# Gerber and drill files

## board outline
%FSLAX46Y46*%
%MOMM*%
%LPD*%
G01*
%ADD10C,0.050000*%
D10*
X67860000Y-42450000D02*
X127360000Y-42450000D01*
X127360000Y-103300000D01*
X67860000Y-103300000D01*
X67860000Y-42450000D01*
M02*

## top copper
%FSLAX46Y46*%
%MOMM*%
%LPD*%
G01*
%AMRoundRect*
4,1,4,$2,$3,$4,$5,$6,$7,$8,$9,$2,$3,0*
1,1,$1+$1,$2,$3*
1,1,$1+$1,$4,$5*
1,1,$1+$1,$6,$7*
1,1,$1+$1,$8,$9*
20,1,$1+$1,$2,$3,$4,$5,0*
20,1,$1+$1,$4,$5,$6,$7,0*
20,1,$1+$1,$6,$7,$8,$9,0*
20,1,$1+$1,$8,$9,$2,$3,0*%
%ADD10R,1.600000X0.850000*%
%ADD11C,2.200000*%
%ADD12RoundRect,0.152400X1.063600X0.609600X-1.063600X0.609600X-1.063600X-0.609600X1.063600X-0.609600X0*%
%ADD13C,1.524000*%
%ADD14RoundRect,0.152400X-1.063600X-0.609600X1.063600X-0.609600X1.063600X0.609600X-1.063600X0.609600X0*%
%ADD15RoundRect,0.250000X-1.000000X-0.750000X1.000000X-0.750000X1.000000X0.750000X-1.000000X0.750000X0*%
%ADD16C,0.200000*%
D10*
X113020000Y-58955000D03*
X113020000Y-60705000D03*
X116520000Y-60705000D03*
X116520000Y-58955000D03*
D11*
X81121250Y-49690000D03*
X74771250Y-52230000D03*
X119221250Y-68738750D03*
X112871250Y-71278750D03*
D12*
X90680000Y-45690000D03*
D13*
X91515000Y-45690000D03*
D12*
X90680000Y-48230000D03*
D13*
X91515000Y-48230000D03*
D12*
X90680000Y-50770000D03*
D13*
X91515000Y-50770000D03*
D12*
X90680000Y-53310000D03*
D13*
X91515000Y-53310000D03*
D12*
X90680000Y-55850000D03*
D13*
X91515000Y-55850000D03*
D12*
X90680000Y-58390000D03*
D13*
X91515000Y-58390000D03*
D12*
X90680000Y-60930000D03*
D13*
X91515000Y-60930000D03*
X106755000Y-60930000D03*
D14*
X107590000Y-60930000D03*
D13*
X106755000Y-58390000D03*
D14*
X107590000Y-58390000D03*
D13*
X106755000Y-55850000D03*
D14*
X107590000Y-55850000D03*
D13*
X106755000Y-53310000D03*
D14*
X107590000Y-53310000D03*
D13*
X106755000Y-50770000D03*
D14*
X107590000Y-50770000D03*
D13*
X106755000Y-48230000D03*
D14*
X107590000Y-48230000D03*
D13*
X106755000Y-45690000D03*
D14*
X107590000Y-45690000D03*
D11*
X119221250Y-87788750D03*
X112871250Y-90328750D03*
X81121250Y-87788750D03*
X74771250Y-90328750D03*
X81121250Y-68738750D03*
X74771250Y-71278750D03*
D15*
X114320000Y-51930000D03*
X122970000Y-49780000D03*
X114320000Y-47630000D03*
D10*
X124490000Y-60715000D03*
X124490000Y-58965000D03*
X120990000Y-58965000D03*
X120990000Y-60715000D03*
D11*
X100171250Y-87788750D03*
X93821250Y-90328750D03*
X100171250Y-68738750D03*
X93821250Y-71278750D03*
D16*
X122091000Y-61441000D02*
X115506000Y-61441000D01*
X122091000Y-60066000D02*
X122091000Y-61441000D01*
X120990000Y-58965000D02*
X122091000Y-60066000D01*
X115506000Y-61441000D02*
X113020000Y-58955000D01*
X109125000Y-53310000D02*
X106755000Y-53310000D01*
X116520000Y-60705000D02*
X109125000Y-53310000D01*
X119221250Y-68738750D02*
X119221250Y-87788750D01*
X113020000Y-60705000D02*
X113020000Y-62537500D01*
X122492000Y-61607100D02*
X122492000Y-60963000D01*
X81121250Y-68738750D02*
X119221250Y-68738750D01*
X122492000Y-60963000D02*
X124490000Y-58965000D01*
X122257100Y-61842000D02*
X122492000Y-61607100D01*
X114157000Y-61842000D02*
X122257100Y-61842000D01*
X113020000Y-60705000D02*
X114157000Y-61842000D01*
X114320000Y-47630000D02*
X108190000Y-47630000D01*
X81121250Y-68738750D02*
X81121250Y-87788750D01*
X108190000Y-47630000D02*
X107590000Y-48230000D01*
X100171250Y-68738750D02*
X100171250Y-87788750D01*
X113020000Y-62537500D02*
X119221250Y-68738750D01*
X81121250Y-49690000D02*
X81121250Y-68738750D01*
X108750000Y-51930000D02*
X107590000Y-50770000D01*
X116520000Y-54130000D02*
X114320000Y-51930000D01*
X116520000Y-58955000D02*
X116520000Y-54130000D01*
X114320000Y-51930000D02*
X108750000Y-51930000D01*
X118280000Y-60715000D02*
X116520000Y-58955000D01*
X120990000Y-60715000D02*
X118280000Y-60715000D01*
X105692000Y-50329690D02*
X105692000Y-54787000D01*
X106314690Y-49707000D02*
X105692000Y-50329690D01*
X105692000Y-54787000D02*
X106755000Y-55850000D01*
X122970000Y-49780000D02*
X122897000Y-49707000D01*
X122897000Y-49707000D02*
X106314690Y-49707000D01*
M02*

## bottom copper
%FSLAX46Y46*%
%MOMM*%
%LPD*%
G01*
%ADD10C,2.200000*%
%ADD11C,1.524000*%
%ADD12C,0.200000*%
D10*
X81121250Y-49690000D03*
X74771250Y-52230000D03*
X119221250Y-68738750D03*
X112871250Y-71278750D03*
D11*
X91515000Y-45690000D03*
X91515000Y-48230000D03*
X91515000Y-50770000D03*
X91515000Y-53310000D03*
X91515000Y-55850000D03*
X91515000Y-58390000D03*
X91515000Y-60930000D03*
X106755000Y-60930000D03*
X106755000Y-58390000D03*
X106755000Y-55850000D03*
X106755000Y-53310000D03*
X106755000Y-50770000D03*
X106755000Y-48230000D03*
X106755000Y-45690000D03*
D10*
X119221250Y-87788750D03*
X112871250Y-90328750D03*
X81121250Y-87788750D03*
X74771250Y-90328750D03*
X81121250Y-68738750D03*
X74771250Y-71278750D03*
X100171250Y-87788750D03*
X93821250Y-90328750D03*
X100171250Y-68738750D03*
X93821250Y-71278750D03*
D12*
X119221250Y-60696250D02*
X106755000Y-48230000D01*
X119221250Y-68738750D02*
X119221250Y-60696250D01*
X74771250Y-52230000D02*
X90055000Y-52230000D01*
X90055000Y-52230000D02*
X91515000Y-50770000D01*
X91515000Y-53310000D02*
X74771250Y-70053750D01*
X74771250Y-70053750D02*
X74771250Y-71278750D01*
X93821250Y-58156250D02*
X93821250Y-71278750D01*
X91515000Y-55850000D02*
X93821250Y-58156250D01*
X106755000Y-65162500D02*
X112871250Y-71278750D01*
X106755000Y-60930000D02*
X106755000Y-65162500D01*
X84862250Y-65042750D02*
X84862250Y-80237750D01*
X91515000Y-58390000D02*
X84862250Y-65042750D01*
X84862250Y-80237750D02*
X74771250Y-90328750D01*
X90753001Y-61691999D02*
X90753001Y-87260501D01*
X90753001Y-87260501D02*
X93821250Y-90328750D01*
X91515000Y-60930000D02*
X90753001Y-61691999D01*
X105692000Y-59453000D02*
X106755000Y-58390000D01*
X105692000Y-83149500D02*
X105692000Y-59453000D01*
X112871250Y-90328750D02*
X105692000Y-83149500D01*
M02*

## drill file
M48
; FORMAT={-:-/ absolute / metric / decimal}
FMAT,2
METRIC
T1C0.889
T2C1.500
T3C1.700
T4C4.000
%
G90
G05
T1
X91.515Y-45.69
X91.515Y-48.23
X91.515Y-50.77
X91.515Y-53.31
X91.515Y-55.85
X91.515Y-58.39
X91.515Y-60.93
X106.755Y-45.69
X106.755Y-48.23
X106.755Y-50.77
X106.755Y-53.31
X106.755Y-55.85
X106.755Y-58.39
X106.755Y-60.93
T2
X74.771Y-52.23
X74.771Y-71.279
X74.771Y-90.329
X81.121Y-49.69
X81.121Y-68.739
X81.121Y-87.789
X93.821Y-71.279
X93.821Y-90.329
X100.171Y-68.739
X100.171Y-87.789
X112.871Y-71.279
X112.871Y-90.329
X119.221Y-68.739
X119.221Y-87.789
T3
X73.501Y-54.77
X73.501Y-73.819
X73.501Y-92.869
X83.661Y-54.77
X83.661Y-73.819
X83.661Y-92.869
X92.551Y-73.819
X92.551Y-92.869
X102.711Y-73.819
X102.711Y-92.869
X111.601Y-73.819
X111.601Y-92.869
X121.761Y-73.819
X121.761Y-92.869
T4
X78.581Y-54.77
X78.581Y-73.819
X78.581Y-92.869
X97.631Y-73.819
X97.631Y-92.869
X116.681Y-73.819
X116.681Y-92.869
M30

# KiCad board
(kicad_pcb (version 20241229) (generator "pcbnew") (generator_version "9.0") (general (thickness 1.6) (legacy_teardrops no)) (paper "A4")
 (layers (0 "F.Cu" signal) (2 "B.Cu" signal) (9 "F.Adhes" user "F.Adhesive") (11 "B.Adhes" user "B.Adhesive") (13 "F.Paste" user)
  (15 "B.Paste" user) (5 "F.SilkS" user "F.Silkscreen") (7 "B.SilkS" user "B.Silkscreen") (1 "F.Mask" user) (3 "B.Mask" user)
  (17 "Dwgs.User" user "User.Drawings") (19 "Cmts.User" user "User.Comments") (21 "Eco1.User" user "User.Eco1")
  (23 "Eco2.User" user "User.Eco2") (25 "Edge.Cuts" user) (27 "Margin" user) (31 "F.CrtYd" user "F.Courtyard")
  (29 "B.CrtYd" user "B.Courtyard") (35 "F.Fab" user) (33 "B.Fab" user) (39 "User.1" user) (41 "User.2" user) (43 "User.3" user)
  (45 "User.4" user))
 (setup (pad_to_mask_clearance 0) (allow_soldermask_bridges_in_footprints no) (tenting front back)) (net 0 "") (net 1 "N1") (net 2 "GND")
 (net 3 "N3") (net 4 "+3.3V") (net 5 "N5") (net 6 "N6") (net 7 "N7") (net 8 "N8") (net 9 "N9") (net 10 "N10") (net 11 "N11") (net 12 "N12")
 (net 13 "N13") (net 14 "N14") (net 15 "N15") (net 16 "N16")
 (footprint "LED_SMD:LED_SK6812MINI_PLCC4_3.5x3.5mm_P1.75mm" (layer "F.Cu") (at 114.77 59.83)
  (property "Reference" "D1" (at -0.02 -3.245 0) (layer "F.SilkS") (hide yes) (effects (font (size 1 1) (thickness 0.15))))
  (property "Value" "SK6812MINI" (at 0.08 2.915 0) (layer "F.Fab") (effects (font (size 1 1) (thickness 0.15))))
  (pad "1" smd rect (at -1.75 -0.875) (size 1.6 0.85) (layers "F.Cu" "F.Mask" "F.Paste") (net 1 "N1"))
  (pad "2" smd rect (at -1.75 0.875) (size 1.6 0.85) (layers "F.Cu" "F.Mask" "F.Paste") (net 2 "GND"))
  (pad "3" smd rect (at 1.75 0.875) (size 1.6 0.85) (layers "F.Cu" "F.Mask" "F.Paste") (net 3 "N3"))
  (pad "4" smd rect (at 1.75 -0.875) (size 1.6 0.85) (layers "F.Cu" "F.Mask" "F.Paste") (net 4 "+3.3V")))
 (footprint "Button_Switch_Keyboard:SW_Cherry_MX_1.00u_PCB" (layer "F.Cu") (at 81.12125 49.69)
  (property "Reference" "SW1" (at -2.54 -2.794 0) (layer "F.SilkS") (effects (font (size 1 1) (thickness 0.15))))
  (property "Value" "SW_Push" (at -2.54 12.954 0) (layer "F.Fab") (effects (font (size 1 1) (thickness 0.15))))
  (pad "" np_thru_hole circle (at -7.62 5.08) (size 1.7 1.7) (drill 1.7) (layers "*.Cu" "*.Mask"))
  (pad "" np_thru_hole circle (at -2.54 5.08) (size 4 4) (drill 4) (layers "*.Cu" "*.Mask"))
  (pad "" np_thru_hole circle (at 2.54 5.08) (size 1.7 1.7) (drill 1.7) (layers "*.Cu" "*.Mask"))
  (pad "1" thru_hole circle (at 0 0) (size 2.2 2.2) (drill 1.5) (layers "*.Cu" "*.Mask") (remove_unused_layers no) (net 2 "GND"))
  (pad "2" thru_hole circle (at -6.35 2.54) (size 2.2 2.2) (drill 1.5) (layers "*.Cu" "*.Mask") (remove_unused_layers no) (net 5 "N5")))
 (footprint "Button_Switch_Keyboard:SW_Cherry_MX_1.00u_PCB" (layer "F.Cu") (at 119.22125 68.73875)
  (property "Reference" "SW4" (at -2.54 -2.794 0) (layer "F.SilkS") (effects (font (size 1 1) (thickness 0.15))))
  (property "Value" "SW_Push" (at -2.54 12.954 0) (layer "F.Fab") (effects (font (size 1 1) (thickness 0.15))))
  (pad "" np_thru_hole circle (at -7.62 5.08) (size 1.7 1.7) (drill 1.7) (layers "*.Cu" "*.Mask"))
  (pad "" np_thru_hole circle (at -2.54 5.08) (size 4 4) (drill 4) (layers "*.Cu" "*.Mask"))
  (pad "" np_thru_hole circle (at 2.54 5.08) (size 1.7 1.7) (drill 1.7) (layers "*.Cu" "*.Mask"))
  (pad "1" thru_hole circle (at 0 0) (size 2.2 2.2) (drill 1.5) (layers "*.Cu" "*.Mask") (remove_unused_layers no) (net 2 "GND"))
  (pad "2" thru_hole circle (at -6.35 2.54) (size 2.2 2.2) (drill 1.5) (layers "*.Cu" "*.Mask") (remove_unused_layers no) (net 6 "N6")))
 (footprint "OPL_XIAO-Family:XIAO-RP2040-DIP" (layer "F.Cu") (at 99.135 53.31)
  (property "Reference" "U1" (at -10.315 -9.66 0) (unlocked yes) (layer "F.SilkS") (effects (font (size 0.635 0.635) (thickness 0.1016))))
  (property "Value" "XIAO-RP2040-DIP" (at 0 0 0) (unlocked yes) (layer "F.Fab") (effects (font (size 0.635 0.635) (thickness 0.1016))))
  (pad "1" smd roundrect (at -8.455 -7.62 180) (size 2.432 1.524) (layers "F.Cu" "F.Mask") (roundrect_rratio 0.1) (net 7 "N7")
   (thermal_bridge_angle 45))
  (pad "1" thru_hole circle (at -7.62 -7.62 180) (size 1.524 1.524) (drill 0.889) (layers "*.Cu" "*.Mask") (remove_unused_layers no)
   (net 7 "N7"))
  (pad "2" smd roundrect (at -8.455 -5.08 180) (size 2.432 1.524) (layers "F.Cu" "F.Mask") (roundrect_rratio 0.1) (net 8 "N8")
   (thermal_bridge_angle 45))
  (pad "2" thru_hole circle (at -7.62 -5.08 180) (size 1.524 1.524) (drill 0.889) (layers "*.Cu" "*.Mask") (remove_unused_layers no)
   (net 8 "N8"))
  (pad "3" smd roundrect (at -8.455 -2.54 180) (size 2.432 1.524) (layers "F.Cu" "F.Mask") (roundrect_rratio 0.1) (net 5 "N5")
   (thermal_bridge_angle 45))
  (pad "3" thru_hole circle (at -7.62 -2.54 180) (size 1.524 1.524) (drill 0.889) (layers "*.Cu" "*.Mask") (remove_unused_layers no)
   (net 5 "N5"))
  (pad "4" smd roundrect (at -8.455 0 180) (size 2.432 1.524) (layers "F.Cu" "F.Mask") (roundrect_rratio 0.1) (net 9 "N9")
   (thermal_bridge_angle 45))
  (pad "4" thru_hole circle (at -7.62 0 180) (size 1.524 1.524) (drill 0.889) (layers "*.Cu" "*.Mask") (remove_unused_layers no)
   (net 9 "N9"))
  (pad "5" smd roundrect (at -8.455 2.54 180) (size 2.432 1.524) (layers "F.Cu" "F.Mask") (roundrect_rratio 0.1) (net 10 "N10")
   (thermal_bridge_angle 45))
  (pad "5" thru_hole circle (at -7.62 2.54 180) (size 1.524 1.524) (drill 0.889) (layers "*.Cu" "*.Mask") (remove_unused_layers no)
   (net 10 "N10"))
  (pad "6" smd roundrect (at -8.455 5.08 180) (size 2.432 1.524) (layers "F.Cu" "F.Mask") (roundrect_rratio 0.1) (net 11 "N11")
   (thermal_bridge_angle 45))
  (pad "6" thru_hole circle (at -7.62 5.08 180) (size 1.524 1.524) (drill 0.889) (layers "*.Cu" "*.Mask") (remove_unused_layers no)
   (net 11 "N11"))
  (pad "7" smd roundrect (at -8.455 7.62 180) (size 2.432 1.524) (layers "F.Cu" "F.Mask") (roundrect_rratio 0.1) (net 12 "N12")
   (thermal_bridge_angle 45))
  (pad "7" thru_hole circle (at -7.62 7.62 180) (size 1.524 1.524) (drill 0.889) (layers "*.Cu" "*.Mask") (remove_unused_layers no)
   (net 12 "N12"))
  (pad "8" thru_hole circle (at 7.62 7.62) (size 1.524 1.524) (drill 0.889) (layers "*.Cu" "*.Mask") (remove_unused_layers no) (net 6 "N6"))
  (pad "8" smd roundrect (at 8.455 7.62) (size 2.432 1.524) (layers "F.Cu" "F.Mask") (roundrect_rratio 0.1) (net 6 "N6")
   (thermal_bridge_angle 45))
  (pad "9" thru_hole circle (at 7.62 5.08) (size 1.524 1.524) (drill 0.889) (layers "*.Cu" "*.Mask") (remove_unused_layers no)
   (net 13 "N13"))
  (pad "9" smd roundrect (at 8.455 5.08) (size 2.432 1.524) (layers "F.Cu" "F.Mask") (roundrect_rratio 0.1) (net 13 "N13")
   (thermal_bridge_angle 45))
  (pad "10" thru_hole circle (at 7.62 2.54) (size 1.524 1.524) (drill 0.889) (layers "*.Cu" "*.Mask") (remove_unused_layers no)
   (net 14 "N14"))
  (pad "10" smd roundrect (at 8.455 2.54) (size 2.432 1.524) (layers "F.Cu" "F.Mask") (roundrect_rratio 0.1) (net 14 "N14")
   (thermal_bridge_angle 45))
  (pad "11" thru_hole circle (at 7.62 0) (size 1.524 1.524) (drill 0.889) (layers "*.Cu" "*.Mask") (remove_unused_layers no) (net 3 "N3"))
  (pad "11" smd roundrect (at 8.455 0) (size 2.432 1.524) (layers "F.Cu" "F.Mask") (roundrect_rratio 0.1) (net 3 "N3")
   (thermal_bridge_angle 45))
  (pad "12" thru_hole circle (at 7.62 -2.54) (size 1.524 1.524) (drill 0.889) (layers "*.Cu" "*.Mask") (remove_unused_layers no)
   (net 4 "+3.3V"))
  (pad "12" smd roundrect (at 8.455 -2.54) (size 2.432 1.524) (layers "F.Cu" "F.Mask") (roundrect_rratio 0.1) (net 4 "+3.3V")
   (thermal_bridge_angle 45))
  (pad "13" thru_hole circle (at 7.62 -5.08) (size 1.524 1.524) (drill 0.889) (layers "*.Cu" "*.Mask") (remove_unused_layers no)
   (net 2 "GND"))
  (pad "13" smd roundrect (at 8.455 -5.08) (size 2.432 1.524) (layers "F.Cu" "F.Mask") (roundrect_rratio 0.1) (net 2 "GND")
   (thermal_bridge_angle 45))
  (pad "14" thru_hole circle (at 7.62 -7.62) (size 1.524 1.524) (drill 0.889) (layers "*.Cu" "*.Mask") (remove_unused_layers no)
   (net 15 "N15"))
  (pad "14" smd roundrect (at 8.455 -7.62) (size 2.432 1.524) (layers "F.Cu" "F.Mask") (roundrect_rratio 0.1) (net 15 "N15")
   (thermal_bridge_angle 45)))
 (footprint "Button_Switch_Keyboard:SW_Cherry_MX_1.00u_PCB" (layer "F.Cu") (at 119.22125 87.78875)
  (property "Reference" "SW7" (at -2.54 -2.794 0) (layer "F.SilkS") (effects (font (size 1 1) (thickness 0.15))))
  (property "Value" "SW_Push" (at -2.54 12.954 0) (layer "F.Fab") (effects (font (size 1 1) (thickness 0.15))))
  (pad "" np_thru_hole circle (at -7.62 5.08) (size 1.7 1.7) (drill 1.7) (layers "*.Cu" "*.Mask"))
  (pad "" np_thru_hole circle (at -2.54 5.08) (size 4 4) (drill 4) (layers "*.Cu" "*.Mask"))
  (pad "" np_thru_hole circle (at 2.54 5.08) (size 1.7 1.7) (drill 1.7) (layers "*.Cu" "*.Mask"))
  (pad "1" thru_hole circle (at 0 0) (size 2.2 2.2) (drill 1.5) (layers "*.Cu" "*.Mask") (remove_unused_layers no) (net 2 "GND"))
  (pad "2" thru_hole circle (at -6.35 2.54) (size 2.2 2.2) (drill 1.5) (layers "*.Cu" "*.Mask") (remove_unused_layers no) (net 13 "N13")))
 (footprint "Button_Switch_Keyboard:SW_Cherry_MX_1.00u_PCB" (layer "F.Cu") (at 81.12125 87.78875)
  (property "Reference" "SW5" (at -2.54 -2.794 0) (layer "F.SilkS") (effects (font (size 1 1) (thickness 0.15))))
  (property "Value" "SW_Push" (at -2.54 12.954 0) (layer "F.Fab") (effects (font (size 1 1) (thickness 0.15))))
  (pad "" np_thru_hole circle (at -7.62 5.08) (size 1.7 1.7) (drill 1.7) (layers "*.Cu" "*.Mask"))
  (pad "" np_thru_hole circle (at -2.54 5.08) (size 4 4) (drill 4) (layers "*.Cu" "*.Mask"))
  (pad "" np_thru_hole circle (at 2.54 5.08) (size 1.7 1.7) (drill 1.7) (layers "*.Cu" "*.Mask"))
  (pad "1" thru_hole circle (at 0 0) (size 2.2 2.2) (drill 1.5) (layers "*.Cu" "*.Mask") (remove_unused_layers no) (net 2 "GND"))
  (pad "2" thru_hole circle (at -6.35 2.54) (size 2.2 2.2) (drill 1.5) (layers "*.Cu" "*.Mask") (remove_unused_layers no) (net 11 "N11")))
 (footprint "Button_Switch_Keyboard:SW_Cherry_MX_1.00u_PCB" (layer "F.Cu") (at 81.12125 68.73875)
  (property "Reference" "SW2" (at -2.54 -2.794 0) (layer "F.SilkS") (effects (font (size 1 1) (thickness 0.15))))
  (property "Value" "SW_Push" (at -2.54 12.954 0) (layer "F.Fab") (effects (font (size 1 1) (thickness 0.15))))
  (pad "" np_thru_hole circle (at -7.62 5.08) (size 1.7 1.7) (drill 1.7) (layers "*.Cu" "*.Mask"))
  (pad "" np_thru_hole circle (at -2.54 5.08) (size 4 4) (drill 4) (layers "*.Cu" "*.Mask"))
  (pad "" np_thru_hole circle (at 2.54 5.08) (size 1.7 1.7) (drill 1.7) (layers "*.Cu" "*.Mask"))
  (pad "1" thru_hole circle (at 0 0) (size 2.2 2.2) (drill 1.5) (layers "*.Cu" "*.Mask") (remove_unused_layers no) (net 2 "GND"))
  (pad "2" thru_hole circle (at -6.35 2.54) (size 2.2 2.2) (drill 1.5) (layers "*.Cu" "*.Mask") (remove_unused_layers no) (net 9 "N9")))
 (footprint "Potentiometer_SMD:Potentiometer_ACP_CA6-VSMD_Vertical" (layer "F.Cu") (at 118.645 49.78)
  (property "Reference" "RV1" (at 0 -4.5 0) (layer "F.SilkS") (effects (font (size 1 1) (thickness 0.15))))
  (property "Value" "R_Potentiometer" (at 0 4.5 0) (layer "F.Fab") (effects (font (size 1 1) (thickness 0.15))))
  (pad "1" smd roundrect (at -4.325 2.15) (size 2.5 2) (layers "F.Cu" "F.Mask" "F.Paste") (roundrect_rratio 0.125) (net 4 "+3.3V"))
  (pad "2" smd roundrect (at 4.325 0) (size 2.5 2) (layers "F.Cu" "F.Mask" "F.Paste") (roundrect_rratio 0.125) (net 14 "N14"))
  (pad "3" smd roundrect (at -4.325 -2.15) (size 2.5 2) (layers "F.Cu" "F.Mask" "F.Paste") (roundrect_rratio 0.125) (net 2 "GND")))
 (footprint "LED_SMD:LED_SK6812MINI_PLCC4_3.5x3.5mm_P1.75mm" (layer "F.Cu") (at 122.74 59.84 180)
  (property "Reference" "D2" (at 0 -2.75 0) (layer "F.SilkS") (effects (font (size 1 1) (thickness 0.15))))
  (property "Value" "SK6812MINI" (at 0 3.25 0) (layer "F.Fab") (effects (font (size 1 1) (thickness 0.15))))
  (pad "1" smd rect (at -1.75 -0.875 180) (size 1.6 0.85) (layers "F.Cu" "F.Mask" "F.Paste") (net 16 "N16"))
  (pad "2" smd rect (at -1.75 0.875 180) (size 1.6 0.85) (layers "F.Cu" "F.Mask" "F.Paste") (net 2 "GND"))
  (pad "3" smd rect (at 1.75 0.875 180) (size 1.6 0.85) (layers "F.Cu" "F.Mask" "F.Paste") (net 1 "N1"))
  (pad "4" smd rect (at 1.75 -0.875 180) (size 1.6 0.85) (layers "F.Cu" "F.Mask" "F.Paste") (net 4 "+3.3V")))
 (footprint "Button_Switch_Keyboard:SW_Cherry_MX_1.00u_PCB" (layer "F.Cu") (at 100.17125 87.78875)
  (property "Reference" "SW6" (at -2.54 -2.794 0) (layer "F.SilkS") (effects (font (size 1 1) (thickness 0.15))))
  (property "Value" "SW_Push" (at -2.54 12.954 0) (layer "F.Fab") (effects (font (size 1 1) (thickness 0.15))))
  (pad "" np_thru_hole circle (at -7.62 5.08) (size 1.7 1.7) (drill 1.7) (layers "*.Cu" "*.Mask"))
  (pad "" np_thru_hole circle (at -2.54 5.08) (size 4 4) (drill 4) (layers "*.Cu" "*.Mask"))
  (pad "" np_thru_hole circle (at 2.54 5.08) (size 1.7 1.7) (drill 1.7) (layers "*.Cu" "*.Mask"))
  (pad "1" thru_hole circle (at 0 0) (size 2.2 2.2) (drill 1.5) (layers "*.Cu" "*.Mask") (remove_unused_layers no) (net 2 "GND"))
  (pad "2" thru_hole circle (at -6.35 2.54) (size 2.2 2.2) (drill 1.5) (layers "*.Cu" "*.Mask") (remove_unused_layers no) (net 12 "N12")))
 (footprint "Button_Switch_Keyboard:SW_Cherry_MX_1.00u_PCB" (layer "F.Cu") (at 100.17125 68.73875)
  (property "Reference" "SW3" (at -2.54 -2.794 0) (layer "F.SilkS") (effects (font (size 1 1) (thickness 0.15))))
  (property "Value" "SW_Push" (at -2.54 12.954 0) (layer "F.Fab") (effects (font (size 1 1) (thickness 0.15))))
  (pad "" np_thru_hole circle (at -7.62 5.08) (size 1.7 1.7) (drill 1.7) (layers "*.Cu" "*.Mask"))
  (pad "" np_thru_hole circle (at -2.54 5.08) (size 4 4) (drill 4) (layers "*.Cu" "*.Mask"))
  (pad "" np_thru_hole circle (at 2.54 5.08) (size 1.7 1.7) (drill 1.7) (layers "*.Cu" "*.Mask"))
  (pad "1" thru_hole circle (at 0 0) (size 2.2 2.2) (drill 1.5) (layers "*.Cu" "*.Mask") (remove_unused_layers no) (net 2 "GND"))
  (pad "2" thru_hole circle (at -6.35 2.54) (size 2.2 2.2) (drill 1.5) (layers "*.Cu" "*.Mask") (remove_unused_layers no) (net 10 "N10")))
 (gr_rect (start 67.86 42.45) (end 127.36 103.3) (stroke (width 0.05) (type default)) (fill no) (layer "Edge.Cuts"))
 (segment (start 122.091 61.441) (end 115.506 61.441) (width 0.2) (layer "F.Cu") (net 1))
 (segment (start 122.091 60.066) (end 122.091 61.441) (width 0.2) (layer "F.Cu") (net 1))
 (segment (start 120.99 58.965) (end 122.091 60.066) (width 0.2) (layer "F.Cu") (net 1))
 (segment (start 115.506 61.441) (end 113.02 58.955) (width 0.2) (layer "F.Cu") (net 1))
 (segment (start 109.125 53.31) (end 106.755 53.31) (width 0.2) (layer "F.Cu") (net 3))
 (segment (start 116.52 60.705) (end 109.125 53.31) (width 0.2) (layer "F.Cu") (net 3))
 (segment (start 119.22125 68.73875) (end 119.22125 87.78875) (width 0.2) (layer "F.Cu") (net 2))
 (segment (start 113.02 60.705) (end 113.02 62.5375) (width 0.2) (layer "F.Cu") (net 2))
 (segment (start 122.492 61.6071) (end 122.492 60.963) (width 0.2) (layer "F.Cu") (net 2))
 (segment (start 81.12125 68.73875) (end 119.22125 68.73875) (width 0.2) (layer "F.Cu") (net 2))
 (segment (start 122.492 60.963) (end 124.49 58.965) (width 0.2) (layer "F.Cu") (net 2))
 (segment (start 122.2571 61.842) (end 122.492 61.6071) (width 0.2) (layer "F.Cu") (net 2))
 (segment (start 114.157 61.842) (end 122.2571 61.842) (width 0.2) (layer "F.Cu") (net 2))
 (segment (start 113.02 60.705) (end 114.157 61.842) (width 0.2) (layer "F.Cu") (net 2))
 (segment (start 114.32 47.63) (end 108.19 47.63) (width 0.2) (layer "F.Cu") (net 2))
 (segment (start 81.12125 68.73875) (end 81.12125 87.78875) (width 0.2) (layer "F.Cu") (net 2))
 (segment (start 108.19 47.63) (end 107.59 48.23) (width 0.2) (layer "F.Cu") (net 2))
 (segment (start 100.17125 68.73875) (end 100.17125 87.78875) (width 0.2) (layer "F.Cu") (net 2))
 (segment (start 113.02 62.5375) (end 119.22125 68.73875) (width 0.2) (layer "F.Cu") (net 2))
 (segment (start 81.12125 49.69) (end 81.12125 68.73875) (width 0.2) (layer "F.Cu") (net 2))
 (segment (start 119.22125 60.69625) (end 106.755 48.23) (width 0.2) (layer "B.Cu") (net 2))
 (segment (start 119.22125 68.73875) (end 119.22125 60.69625) (width 0.2) (layer "B.Cu") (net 2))
 (segment (start 108.75 51.93) (end 107.59 50.77) (width 0.2) (layer "F.Cu") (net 4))
 (segment (start 116.52 54.13) (end 114.32 51.93) (width 0.2) (layer "F.Cu") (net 4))
 (segment (start 116.52 58.955) (end 116.52 54.13) (width 0.2) (layer "F.Cu") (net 4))
 (segment (start 114.32 51.93) (end 108.75 51.93) (width 0.2) (layer "F.Cu") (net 4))
 (segment (start 118.28 60.715) (end 116.52 58.955) (width 0.2) (layer "F.Cu") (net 4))
 (segment (start 120.99 60.715) (end 118.28 60.715) (width 0.2) (layer "F.Cu") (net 4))
 (segment (start 105.692 50.32969) (end 105.692 54.787) (width 0.2) (layer "F.Cu") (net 14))
 (segment (start 106.31469 49.707) (end 105.692 50.32969) (width 0.2) (layer "F.Cu") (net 14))
 (segment (start 105.692 54.787) (end 106.755 55.85) (width 0.2) (layer "F.Cu") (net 14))
 (segment (start 122.97 49.78) (end 122.897 49.707) (width 0.2) (layer "F.Cu") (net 14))
 (segment (start 122.897 49.707) (end 106.31469 49.707) (width 0.2) (layer "F.Cu") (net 14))
 (segment (start 74.77125 52.23) (end 90.055 52.23) (width 0.2) (layer "B.Cu") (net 5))
 (segment (start 90.055 52.23) (end 91.515 50.77) (width 0.2) (layer "B.Cu") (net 5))
 (segment (start 91.515 53.31) (end 74.77125 70.05375) (width 0.2) (layer "B.Cu") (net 9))
 (segment (start 74.77125 70.05375) (end 74.77125 71.27875) (width 0.2) (layer "B.Cu") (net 9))
 (segment (start 93.82125 58.15625) (end 93.82125 71.27875) (width 0.2) (layer "B.Cu") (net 10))
 (segment (start 91.515 55.85) (end 93.82125 58.15625) (width 0.2) (layer "B.Cu") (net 10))
 (segment (start 106.755 65.1625) (end 112.87125 71.27875) (width 0.2) (layer "B.Cu") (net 6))
 (segment (start 106.755 60.93) (end 106.755 65.1625) (width 0.2) (layer "B.Cu") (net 6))
 (segment (start 84.86225 65.04275) (end 84.86225 80.23775) (width 0.2) (layer "B.Cu") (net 11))
 (segment (start 91.515 58.39) (end 84.86225 65.04275) (width 0.2) (layer "B.Cu") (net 11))
 (segment (start 84.86225 80.23775) (end 74.77125 90.32875) (width 0.2) (layer "B.Cu") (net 11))
 (segment (start 90.753001 61.691999) (end 90.753001 87.260501) (width 0.2) (layer "B.Cu") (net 12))
 (segment (start 90.753001 87.260501) (end 93.82125 90.32875) (width 0.2) (layer "B.Cu") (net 12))
 (segment (start 91.515 60.93) (end 90.753001 61.691999) (width 0.2) (layer "B.Cu") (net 12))
 (segment (start 105.692 59.453) (end 106.755 58.39) (width 0.2) (layer "B.Cu") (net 13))
 (segment (start 105.692 83.1495) (end 105.692 59.453) (width 0.2) (layer "B.Cu") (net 13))
 (segment (start 112.87125 90.32875) (end 105.692 83.1495) (width 0.2) (layer "B.Cu") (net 13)))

